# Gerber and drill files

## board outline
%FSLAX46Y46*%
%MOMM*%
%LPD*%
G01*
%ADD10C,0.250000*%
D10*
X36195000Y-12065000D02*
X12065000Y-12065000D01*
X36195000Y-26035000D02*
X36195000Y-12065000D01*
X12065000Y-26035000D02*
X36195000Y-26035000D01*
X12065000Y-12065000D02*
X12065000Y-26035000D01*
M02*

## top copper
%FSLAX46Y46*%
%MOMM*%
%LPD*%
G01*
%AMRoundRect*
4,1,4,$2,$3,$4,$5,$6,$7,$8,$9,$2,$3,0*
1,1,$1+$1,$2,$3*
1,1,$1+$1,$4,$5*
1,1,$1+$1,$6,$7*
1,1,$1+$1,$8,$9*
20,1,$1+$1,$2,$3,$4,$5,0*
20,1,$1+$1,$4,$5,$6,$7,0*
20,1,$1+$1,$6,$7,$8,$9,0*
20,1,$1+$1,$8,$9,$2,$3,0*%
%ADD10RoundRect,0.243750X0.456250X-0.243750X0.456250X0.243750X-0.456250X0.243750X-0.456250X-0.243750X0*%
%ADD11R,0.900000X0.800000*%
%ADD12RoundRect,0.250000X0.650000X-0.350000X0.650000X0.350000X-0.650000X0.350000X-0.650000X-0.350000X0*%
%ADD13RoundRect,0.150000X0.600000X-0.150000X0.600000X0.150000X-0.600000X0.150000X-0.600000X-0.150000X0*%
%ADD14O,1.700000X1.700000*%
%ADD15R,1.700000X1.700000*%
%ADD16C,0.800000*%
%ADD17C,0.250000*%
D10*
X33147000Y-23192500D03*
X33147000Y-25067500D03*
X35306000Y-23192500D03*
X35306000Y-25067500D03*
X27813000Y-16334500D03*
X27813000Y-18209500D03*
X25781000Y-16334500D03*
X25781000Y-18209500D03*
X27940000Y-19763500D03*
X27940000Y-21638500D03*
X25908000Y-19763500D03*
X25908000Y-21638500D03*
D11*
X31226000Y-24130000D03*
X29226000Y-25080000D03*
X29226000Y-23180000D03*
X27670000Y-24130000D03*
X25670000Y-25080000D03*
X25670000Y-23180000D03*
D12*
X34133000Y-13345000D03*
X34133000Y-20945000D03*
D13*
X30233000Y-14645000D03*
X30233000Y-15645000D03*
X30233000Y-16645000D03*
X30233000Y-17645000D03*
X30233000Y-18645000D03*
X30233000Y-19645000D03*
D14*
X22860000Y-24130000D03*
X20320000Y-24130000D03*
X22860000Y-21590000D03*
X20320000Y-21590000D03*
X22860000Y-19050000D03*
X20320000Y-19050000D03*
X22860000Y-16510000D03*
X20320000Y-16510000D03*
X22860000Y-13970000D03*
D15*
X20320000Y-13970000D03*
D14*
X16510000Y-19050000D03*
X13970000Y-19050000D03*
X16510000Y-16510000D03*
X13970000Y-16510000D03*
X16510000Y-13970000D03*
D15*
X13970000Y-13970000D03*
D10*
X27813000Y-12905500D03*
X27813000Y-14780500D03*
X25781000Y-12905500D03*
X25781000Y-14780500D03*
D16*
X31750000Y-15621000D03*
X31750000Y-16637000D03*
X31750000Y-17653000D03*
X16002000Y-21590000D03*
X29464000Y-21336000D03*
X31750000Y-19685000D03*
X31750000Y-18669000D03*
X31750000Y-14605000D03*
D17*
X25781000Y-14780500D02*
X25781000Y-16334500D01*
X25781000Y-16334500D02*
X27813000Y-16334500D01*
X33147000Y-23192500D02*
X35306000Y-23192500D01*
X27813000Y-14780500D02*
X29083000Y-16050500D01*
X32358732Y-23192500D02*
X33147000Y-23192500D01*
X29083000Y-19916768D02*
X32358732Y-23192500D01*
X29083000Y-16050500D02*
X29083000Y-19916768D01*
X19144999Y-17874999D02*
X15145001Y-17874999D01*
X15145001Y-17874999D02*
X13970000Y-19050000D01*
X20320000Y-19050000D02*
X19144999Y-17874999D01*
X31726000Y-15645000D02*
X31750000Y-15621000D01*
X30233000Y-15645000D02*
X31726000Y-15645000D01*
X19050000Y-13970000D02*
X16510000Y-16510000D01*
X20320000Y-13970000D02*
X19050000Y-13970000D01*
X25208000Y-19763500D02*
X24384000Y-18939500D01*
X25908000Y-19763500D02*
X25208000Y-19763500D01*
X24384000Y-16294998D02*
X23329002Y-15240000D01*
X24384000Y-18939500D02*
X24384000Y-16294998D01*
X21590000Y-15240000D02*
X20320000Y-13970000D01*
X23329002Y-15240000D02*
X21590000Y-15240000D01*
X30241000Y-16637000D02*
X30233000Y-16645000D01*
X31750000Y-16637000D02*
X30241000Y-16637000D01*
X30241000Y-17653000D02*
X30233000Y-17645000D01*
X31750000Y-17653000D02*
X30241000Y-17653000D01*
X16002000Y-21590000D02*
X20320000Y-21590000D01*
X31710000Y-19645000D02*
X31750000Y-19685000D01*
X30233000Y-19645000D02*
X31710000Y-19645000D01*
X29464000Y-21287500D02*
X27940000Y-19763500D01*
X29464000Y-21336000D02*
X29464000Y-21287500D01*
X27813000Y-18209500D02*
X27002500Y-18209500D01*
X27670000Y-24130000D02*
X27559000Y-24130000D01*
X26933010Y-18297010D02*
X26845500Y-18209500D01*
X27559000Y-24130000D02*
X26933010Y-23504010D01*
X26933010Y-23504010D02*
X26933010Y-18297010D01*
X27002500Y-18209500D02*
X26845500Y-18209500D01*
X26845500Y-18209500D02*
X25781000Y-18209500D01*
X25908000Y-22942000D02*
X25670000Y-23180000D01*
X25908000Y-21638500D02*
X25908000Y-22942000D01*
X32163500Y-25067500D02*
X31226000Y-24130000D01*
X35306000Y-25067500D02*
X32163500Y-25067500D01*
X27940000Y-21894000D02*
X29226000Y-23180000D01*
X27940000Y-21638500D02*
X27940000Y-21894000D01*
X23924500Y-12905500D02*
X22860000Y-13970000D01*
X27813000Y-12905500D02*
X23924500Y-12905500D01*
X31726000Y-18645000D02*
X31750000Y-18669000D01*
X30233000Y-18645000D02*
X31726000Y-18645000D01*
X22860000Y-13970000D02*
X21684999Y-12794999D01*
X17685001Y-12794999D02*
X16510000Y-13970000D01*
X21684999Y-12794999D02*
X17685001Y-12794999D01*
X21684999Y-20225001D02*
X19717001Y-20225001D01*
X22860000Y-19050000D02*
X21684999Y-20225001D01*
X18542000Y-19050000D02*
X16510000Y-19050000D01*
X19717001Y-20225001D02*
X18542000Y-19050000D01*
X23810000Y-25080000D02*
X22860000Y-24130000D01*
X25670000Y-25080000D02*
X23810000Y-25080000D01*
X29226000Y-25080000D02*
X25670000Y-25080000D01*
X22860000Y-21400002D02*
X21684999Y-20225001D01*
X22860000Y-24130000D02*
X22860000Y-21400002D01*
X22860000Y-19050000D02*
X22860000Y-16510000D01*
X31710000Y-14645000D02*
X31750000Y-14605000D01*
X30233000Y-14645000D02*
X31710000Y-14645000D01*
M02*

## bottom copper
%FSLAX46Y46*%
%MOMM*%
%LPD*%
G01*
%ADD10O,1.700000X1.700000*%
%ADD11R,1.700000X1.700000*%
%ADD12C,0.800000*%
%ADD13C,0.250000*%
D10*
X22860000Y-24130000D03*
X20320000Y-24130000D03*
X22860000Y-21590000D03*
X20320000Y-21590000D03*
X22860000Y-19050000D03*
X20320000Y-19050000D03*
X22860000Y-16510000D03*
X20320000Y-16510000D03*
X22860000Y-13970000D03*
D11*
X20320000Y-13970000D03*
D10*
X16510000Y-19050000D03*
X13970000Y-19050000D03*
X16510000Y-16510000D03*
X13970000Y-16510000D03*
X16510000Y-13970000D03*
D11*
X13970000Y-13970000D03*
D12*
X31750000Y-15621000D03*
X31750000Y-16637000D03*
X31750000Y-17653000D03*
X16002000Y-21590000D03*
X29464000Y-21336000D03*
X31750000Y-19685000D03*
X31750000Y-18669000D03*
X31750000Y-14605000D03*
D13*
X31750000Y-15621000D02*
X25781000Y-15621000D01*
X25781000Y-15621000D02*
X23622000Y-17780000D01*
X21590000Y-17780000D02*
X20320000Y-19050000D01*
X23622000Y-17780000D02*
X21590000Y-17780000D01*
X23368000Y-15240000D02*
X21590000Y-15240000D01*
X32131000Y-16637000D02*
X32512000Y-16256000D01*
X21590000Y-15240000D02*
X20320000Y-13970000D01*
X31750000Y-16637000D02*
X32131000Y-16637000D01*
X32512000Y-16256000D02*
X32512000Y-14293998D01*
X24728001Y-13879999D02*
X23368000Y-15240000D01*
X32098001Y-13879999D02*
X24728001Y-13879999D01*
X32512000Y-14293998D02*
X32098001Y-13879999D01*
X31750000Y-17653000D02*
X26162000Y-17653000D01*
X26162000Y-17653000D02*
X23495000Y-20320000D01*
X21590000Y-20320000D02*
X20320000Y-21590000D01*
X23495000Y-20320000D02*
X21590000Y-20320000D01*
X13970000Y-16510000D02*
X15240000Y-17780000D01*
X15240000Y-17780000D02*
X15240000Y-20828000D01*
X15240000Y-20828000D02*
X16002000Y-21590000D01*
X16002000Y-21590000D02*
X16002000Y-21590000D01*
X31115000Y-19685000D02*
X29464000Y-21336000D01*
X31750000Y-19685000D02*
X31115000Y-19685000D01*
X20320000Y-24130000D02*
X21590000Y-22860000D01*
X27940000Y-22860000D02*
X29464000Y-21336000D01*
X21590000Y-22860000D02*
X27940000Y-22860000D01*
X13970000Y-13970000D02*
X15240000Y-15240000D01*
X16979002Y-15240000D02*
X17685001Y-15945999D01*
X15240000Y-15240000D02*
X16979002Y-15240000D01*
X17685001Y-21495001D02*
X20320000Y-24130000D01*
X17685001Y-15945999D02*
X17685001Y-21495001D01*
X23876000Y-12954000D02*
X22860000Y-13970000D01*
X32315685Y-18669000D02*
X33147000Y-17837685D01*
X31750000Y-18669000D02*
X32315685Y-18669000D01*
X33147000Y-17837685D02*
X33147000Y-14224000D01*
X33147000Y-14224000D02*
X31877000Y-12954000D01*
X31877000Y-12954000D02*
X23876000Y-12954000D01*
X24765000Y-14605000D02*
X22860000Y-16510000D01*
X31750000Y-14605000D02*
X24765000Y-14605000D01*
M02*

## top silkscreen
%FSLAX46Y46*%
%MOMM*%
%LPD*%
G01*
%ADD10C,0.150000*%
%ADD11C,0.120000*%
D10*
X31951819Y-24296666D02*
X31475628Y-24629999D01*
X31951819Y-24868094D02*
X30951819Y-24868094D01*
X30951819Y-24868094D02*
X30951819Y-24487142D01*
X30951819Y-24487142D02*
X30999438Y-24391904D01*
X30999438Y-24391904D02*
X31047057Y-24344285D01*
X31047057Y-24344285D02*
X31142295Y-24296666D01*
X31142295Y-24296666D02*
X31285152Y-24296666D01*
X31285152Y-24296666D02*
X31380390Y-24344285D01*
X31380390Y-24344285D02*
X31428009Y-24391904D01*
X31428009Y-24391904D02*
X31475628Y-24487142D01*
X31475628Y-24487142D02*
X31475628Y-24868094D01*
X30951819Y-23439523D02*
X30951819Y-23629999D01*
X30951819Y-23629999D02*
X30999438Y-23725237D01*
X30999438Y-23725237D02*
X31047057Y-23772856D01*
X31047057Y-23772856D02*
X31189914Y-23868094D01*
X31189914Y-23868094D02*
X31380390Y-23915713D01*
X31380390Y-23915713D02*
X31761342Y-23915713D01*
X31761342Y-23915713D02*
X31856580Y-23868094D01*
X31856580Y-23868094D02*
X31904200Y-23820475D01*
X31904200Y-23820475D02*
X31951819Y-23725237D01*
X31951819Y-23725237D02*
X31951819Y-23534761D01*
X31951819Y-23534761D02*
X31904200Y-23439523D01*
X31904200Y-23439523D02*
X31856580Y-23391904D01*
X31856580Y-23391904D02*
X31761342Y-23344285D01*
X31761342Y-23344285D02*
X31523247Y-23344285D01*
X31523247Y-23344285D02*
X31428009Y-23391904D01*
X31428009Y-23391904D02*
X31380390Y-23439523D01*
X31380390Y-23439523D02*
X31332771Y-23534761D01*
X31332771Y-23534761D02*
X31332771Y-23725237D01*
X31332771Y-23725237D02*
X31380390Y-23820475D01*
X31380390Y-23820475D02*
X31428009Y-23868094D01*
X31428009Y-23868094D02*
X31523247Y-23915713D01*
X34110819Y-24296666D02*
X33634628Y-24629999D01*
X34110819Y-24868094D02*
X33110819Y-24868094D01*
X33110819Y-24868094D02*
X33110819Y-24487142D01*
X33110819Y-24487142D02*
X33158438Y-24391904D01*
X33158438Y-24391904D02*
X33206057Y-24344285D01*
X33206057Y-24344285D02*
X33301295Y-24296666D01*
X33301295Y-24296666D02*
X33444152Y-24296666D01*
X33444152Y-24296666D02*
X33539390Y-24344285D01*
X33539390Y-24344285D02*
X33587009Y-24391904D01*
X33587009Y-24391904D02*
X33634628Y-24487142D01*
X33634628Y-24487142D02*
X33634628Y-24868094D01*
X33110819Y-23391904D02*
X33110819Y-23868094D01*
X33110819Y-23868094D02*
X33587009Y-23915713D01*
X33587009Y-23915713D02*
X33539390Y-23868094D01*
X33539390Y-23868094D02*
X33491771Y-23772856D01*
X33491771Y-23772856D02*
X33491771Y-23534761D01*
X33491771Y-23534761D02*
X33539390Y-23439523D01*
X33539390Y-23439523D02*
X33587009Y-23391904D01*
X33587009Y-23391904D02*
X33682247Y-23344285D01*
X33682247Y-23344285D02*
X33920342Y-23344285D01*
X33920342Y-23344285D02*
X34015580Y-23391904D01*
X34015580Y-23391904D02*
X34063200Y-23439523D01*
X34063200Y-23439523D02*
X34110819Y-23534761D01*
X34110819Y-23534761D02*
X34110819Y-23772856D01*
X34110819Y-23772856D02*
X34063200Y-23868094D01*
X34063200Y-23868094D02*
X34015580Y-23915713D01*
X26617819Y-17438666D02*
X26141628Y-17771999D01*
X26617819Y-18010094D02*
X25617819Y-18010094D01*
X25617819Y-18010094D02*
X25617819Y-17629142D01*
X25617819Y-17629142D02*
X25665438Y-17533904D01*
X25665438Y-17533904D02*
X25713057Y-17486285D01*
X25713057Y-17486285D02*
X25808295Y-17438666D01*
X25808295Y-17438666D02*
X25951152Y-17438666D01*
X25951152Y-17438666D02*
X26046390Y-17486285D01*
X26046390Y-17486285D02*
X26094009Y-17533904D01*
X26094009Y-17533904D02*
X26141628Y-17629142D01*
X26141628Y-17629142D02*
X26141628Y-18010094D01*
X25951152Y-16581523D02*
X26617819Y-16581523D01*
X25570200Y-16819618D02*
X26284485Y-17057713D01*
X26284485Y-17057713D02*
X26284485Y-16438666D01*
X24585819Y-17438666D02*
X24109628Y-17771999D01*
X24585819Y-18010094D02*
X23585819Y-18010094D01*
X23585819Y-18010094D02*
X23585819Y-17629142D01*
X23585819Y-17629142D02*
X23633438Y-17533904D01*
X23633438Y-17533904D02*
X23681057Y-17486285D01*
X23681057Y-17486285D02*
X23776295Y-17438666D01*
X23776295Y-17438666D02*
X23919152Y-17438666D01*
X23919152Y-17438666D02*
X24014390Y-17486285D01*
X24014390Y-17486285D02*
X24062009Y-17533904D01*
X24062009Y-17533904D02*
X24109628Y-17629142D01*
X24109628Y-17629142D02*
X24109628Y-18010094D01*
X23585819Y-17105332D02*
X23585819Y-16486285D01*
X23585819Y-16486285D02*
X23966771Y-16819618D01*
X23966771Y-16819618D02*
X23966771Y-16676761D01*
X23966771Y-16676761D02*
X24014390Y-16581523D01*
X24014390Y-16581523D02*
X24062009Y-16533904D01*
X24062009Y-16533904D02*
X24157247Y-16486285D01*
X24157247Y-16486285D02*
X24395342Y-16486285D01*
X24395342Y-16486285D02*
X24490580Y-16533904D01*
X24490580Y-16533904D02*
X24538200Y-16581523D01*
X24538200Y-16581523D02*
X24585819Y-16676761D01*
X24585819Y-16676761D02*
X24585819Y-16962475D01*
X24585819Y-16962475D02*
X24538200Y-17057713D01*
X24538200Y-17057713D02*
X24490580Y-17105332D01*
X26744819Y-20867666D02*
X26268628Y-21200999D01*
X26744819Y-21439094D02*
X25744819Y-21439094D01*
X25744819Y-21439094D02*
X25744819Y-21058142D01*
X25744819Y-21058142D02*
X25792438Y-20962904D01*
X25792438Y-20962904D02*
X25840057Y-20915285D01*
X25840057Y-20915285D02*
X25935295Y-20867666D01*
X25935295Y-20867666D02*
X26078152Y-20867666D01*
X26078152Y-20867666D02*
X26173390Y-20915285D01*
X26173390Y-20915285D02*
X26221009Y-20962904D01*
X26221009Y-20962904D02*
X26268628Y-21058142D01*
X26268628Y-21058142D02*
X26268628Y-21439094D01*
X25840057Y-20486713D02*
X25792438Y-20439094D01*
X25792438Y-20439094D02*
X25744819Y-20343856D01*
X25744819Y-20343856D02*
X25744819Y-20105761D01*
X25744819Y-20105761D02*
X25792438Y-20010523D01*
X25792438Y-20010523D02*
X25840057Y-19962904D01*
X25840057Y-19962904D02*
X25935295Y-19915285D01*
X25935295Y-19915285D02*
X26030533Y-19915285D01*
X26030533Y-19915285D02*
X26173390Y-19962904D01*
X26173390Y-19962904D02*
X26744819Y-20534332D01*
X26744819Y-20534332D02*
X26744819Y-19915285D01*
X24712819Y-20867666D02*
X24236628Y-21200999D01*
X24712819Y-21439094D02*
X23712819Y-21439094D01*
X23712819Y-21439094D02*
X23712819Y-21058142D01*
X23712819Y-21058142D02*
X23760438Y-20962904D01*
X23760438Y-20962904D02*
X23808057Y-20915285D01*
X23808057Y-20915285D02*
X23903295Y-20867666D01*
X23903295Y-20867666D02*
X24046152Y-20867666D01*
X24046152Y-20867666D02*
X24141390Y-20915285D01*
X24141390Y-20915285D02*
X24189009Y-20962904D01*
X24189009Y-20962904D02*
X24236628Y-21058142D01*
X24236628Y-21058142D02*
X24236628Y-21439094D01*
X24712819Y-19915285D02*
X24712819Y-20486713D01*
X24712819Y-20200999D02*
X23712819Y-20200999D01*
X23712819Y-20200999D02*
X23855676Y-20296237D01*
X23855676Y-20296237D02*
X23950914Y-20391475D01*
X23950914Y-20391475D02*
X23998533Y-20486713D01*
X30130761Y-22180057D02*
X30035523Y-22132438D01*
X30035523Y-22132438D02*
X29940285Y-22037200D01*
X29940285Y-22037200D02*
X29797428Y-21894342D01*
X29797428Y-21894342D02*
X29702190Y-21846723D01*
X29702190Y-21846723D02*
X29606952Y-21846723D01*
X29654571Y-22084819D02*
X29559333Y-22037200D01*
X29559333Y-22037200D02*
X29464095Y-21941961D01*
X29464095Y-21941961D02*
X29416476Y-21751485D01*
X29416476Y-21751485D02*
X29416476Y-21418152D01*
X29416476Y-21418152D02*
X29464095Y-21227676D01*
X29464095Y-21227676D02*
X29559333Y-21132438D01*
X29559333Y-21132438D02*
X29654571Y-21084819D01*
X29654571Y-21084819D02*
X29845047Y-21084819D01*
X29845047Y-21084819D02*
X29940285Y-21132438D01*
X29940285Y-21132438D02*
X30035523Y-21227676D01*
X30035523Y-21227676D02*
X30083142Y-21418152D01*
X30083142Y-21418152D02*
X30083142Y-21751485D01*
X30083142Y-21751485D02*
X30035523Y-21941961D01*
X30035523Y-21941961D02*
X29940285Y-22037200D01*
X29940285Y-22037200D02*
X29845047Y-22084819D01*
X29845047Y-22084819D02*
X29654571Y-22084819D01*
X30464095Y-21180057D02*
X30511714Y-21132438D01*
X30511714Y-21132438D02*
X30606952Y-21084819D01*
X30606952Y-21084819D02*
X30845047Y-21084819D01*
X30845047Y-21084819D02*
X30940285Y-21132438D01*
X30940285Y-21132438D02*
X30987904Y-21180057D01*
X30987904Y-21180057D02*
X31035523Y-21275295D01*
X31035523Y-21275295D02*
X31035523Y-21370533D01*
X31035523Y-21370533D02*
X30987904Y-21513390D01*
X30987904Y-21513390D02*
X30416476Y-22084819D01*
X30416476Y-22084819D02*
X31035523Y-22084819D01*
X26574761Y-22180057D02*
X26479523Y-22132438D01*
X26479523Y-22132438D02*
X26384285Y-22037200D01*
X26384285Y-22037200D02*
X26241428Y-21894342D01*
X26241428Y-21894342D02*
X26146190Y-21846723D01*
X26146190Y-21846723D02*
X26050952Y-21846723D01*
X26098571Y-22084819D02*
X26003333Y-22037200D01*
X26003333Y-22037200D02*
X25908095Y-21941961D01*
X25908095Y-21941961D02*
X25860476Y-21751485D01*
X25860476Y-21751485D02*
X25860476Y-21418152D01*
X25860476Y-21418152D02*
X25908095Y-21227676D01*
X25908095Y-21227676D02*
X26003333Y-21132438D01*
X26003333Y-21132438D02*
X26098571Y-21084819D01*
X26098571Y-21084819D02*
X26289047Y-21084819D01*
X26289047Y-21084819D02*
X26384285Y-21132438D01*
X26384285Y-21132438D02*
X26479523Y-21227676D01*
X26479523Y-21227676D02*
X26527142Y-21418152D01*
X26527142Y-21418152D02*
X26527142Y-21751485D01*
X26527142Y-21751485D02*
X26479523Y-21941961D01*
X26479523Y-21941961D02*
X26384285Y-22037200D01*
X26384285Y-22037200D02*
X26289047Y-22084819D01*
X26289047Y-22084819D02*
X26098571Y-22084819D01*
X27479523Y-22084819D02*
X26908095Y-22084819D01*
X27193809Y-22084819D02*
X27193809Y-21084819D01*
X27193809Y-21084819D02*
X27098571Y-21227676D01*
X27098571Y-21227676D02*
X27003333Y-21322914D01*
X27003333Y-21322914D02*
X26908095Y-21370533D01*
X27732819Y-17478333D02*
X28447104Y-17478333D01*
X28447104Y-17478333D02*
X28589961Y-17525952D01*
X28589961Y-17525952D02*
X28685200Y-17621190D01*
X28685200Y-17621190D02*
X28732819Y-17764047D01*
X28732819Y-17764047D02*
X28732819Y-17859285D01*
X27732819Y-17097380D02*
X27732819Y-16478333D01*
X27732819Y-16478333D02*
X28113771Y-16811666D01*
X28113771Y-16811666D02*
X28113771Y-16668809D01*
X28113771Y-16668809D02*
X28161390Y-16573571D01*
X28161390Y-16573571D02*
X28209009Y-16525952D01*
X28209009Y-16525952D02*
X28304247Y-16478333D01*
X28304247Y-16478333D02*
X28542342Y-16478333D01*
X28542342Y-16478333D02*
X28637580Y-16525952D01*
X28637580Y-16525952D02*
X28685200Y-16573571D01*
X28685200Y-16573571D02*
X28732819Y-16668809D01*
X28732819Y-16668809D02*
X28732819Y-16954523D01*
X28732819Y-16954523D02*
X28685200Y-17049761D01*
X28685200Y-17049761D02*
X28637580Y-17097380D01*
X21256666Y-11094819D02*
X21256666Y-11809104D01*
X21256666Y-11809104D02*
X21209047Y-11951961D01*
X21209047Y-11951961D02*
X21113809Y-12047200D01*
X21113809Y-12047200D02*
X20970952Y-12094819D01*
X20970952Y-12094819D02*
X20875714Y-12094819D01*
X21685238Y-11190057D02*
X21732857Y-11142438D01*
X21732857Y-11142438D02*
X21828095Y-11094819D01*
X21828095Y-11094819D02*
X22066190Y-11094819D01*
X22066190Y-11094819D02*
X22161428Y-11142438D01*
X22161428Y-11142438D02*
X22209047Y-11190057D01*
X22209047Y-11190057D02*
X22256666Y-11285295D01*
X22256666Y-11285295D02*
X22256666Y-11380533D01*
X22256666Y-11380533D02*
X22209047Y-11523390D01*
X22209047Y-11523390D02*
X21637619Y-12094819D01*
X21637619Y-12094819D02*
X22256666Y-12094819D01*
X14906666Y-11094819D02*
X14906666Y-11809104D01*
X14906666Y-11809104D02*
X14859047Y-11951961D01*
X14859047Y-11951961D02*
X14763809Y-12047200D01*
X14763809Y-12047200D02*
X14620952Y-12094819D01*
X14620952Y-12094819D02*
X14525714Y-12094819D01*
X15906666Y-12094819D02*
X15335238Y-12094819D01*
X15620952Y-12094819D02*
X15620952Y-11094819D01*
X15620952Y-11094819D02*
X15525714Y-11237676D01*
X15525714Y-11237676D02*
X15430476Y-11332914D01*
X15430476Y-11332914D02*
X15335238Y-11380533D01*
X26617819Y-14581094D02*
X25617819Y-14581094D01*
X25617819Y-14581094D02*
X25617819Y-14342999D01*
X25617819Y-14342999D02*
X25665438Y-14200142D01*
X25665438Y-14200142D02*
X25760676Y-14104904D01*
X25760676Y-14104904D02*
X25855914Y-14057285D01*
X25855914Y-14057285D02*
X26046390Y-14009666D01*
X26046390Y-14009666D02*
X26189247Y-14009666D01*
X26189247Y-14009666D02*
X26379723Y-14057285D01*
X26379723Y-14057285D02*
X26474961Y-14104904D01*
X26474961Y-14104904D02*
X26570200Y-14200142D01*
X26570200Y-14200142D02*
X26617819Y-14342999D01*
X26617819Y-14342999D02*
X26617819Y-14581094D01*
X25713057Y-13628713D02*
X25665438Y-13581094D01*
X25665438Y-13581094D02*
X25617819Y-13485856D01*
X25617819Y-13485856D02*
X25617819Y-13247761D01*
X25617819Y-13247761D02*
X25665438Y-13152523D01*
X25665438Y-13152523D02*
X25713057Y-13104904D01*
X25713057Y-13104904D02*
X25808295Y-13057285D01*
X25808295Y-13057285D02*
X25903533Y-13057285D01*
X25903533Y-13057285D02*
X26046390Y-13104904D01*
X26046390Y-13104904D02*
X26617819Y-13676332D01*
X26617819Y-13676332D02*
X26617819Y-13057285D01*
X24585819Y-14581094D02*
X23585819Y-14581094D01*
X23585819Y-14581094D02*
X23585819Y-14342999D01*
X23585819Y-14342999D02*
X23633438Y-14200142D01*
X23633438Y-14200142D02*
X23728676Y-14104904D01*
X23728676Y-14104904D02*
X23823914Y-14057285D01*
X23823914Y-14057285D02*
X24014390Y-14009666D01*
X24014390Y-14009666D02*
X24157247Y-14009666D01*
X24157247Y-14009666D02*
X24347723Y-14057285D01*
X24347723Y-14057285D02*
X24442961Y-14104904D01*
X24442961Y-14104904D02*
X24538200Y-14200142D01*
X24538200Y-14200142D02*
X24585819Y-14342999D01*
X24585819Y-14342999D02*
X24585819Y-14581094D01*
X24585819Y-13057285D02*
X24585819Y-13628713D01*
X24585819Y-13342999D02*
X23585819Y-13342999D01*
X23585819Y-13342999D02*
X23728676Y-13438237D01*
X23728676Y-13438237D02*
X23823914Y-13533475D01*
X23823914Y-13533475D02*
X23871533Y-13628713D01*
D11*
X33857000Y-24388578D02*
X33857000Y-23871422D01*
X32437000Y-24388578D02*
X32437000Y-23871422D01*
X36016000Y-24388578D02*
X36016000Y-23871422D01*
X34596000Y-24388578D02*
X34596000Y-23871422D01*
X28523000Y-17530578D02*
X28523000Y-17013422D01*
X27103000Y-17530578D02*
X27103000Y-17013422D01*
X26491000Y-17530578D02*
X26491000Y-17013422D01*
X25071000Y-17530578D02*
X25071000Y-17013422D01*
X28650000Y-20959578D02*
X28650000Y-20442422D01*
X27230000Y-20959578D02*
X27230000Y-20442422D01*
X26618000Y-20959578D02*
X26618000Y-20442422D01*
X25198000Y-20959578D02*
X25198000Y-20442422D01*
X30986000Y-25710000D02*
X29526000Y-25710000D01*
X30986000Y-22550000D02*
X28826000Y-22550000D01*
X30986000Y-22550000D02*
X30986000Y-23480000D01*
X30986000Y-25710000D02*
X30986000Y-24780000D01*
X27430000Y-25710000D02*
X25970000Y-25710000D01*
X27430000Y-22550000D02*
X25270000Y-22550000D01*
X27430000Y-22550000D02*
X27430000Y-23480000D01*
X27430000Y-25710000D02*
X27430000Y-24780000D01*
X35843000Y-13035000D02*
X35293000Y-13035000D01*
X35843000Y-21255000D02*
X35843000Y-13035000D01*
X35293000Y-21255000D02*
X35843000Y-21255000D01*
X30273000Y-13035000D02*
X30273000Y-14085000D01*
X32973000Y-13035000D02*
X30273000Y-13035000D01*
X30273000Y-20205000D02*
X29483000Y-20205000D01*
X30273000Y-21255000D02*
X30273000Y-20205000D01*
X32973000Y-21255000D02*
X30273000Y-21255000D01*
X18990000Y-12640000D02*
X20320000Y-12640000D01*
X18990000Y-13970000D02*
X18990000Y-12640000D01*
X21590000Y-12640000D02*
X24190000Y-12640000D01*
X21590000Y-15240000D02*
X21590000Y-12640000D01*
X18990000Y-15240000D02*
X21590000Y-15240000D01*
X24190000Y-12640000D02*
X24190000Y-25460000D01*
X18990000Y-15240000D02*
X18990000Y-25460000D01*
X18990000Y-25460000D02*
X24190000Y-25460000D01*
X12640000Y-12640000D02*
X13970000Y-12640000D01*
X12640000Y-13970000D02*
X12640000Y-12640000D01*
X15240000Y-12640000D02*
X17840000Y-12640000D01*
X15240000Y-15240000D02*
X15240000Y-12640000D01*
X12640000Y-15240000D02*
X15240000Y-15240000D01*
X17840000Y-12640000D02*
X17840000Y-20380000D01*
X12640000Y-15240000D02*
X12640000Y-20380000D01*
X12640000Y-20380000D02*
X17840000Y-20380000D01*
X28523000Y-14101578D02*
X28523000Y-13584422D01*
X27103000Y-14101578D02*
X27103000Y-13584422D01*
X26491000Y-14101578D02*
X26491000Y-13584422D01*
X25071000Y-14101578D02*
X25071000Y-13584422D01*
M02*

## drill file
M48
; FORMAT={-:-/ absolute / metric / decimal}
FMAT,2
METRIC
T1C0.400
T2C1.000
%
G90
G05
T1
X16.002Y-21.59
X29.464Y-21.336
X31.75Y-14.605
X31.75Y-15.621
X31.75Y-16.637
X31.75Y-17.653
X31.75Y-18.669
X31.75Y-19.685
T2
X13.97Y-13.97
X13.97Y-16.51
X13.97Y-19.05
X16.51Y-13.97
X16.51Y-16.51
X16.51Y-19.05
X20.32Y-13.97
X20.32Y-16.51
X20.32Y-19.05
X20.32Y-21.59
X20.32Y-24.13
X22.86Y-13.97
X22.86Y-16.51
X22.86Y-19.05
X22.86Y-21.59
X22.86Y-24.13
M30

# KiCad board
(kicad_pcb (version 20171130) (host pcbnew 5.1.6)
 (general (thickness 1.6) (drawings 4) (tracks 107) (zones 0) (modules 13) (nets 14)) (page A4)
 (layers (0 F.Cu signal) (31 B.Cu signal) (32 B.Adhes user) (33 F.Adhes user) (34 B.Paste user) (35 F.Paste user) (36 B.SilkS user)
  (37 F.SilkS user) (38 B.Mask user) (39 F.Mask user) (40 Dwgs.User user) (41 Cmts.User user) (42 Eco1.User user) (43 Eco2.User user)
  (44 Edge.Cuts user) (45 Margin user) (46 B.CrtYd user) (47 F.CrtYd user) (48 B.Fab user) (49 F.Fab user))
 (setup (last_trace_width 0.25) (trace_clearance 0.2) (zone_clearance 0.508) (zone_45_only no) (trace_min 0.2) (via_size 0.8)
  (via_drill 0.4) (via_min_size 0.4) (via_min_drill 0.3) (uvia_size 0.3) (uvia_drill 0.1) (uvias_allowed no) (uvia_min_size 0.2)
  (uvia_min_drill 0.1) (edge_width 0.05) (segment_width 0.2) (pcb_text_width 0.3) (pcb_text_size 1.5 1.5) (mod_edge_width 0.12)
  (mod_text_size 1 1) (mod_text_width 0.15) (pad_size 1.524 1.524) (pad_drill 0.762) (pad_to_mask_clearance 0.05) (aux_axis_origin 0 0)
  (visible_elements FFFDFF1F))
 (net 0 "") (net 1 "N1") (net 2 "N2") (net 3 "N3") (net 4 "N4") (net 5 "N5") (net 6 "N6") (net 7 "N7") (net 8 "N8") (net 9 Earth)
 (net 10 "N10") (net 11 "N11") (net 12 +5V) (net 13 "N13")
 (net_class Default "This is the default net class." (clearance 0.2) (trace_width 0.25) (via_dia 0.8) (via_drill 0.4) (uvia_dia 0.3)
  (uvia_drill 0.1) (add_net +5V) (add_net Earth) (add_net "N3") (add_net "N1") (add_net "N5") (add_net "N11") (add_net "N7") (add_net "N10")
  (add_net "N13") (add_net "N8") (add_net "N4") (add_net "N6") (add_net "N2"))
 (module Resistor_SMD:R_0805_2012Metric (layer F.Cu) (at 33.147 24.13 90)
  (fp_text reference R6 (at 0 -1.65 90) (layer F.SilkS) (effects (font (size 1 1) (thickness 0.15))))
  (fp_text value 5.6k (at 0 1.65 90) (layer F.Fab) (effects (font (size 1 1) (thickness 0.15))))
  (fp_line (start -0.258578 0.71) (end 0.258578 0.71) (layer F.SilkS) (width 0.12))
  (fp_line (start -0.258578 -0.71) (end 0.258578 -0.71) (layer F.SilkS) (width 0.12))
  (pad 2 smd roundrect (at 0.9375 0 90) (size 0.975 1.4) (layers F.Cu F.Paste F.Mask) (roundrect_rratio 0.25) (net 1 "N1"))
  (pad 1 smd roundrect (at -0.9375 0 90) (size 0.975 1.4) (layers F.Cu F.Paste F.Mask) (roundrect_rratio 0.25) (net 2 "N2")))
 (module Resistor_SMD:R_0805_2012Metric (layer F.Cu) (at 35.306 24.13 90)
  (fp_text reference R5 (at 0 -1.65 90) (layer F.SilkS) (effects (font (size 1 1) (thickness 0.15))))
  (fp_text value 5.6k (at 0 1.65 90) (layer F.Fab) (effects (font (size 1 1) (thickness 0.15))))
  (fp_line (start -0.258578 0.71) (end 0.258578 0.71) (layer F.SilkS) (width 0.12))
  (fp_line (start -0.258578 -0.71) (end 0.258578 -0.71) (layer F.SilkS) (width 0.12))
  (pad 2 smd roundrect (at 0.9375 0 90) (size 0.975 1.4) (layers F.Cu F.Paste F.Mask) (roundrect_rratio 0.25) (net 1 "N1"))
  (pad 1 smd roundrect (at -0.9375 0 90) (size 0.975 1.4) (layers F.Cu F.Paste F.Mask) (roundrect_rratio 0.25) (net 2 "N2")))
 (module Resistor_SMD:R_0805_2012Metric (layer F.Cu) (at 27.813 17.272 90)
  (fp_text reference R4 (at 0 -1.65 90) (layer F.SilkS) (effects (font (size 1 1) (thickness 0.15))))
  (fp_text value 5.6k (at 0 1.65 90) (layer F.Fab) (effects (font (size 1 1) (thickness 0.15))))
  (fp_line (start -0.258578 0.71) (end 0.258578 0.71) (layer F.SilkS) (width 0.12))
  (fp_line (start -0.258578 -0.71) (end 0.258578 -0.71) (layer F.SilkS) (width 0.12))
  (pad 2 smd roundrect (at 0.9375 0 90) (size 0.975 1.4) (layers F.Cu F.Paste F.Mask) (roundrect_rratio 0.25) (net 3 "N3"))
  (pad 1 smd roundrect (at -0.9375 0 90) (size 0.975 1.4) (layers F.Cu F.Paste F.Mask) (roundrect_rratio 0.25) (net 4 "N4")))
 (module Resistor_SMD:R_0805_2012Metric (layer F.Cu) (at 25.781 17.272 90)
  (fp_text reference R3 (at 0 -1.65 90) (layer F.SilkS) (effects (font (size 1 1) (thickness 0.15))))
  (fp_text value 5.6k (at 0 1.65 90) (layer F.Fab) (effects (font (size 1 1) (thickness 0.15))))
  (fp_line (start -0.258578 0.71) (end 0.258578 0.71) (layer F.SilkS) (width 0.12))
  (fp_line (start -0.258578 -0.71) (end 0.258578 -0.71) (layer F.SilkS) (width 0.12))
  (pad 2 smd roundrect (at 0.9375 0 90) (size 0.975 1.4) (layers F.Cu F.Paste F.Mask) (roundrect_rratio 0.25) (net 3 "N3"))
  (pad 1 smd roundrect (at -0.9375 0 90) (size 0.975 1.4) (layers F.Cu F.Paste F.Mask) (roundrect_rratio 0.25) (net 4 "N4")))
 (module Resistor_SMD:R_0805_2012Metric (layer F.Cu) (at 27.94 20.701 90)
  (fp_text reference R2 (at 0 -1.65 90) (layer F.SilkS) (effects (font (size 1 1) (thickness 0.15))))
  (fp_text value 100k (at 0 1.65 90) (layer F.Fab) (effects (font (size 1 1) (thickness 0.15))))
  (fp_line (start -0.258578 0.71) (end 0.258578 0.71) (layer F.SilkS) (width 0.12))
  (fp_line (start -0.258578 -0.71) (end 0.258578 -0.71) (layer F.SilkS) (width 0.12))
  (pad 2 smd roundrect (at 0.9375 0 90) (size 0.975 1.4) (layers F.Cu F.Paste F.Mask) (roundrect_rratio 0.25) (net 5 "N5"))
  (pad 1 smd roundrect (at -0.9375 0 90) (size 0.975 1.4) (layers F.Cu F.Paste F.Mask) (roundrect_rratio 0.25) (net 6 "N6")))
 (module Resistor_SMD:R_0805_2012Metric (layer F.Cu) (at 25.908 20.701 90)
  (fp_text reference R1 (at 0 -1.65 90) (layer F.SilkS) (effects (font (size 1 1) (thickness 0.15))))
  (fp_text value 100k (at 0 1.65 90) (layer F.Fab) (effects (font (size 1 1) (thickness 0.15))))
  (fp_line (start -0.258578 0.71) (end 0.258578 0.71) (layer F.SilkS) (width 0.12))
  (fp_line (start -0.258578 -0.71) (end 0.258578 -0.71) (layer F.SilkS) (width 0.12))
  (pad 2 smd roundrect (at 0.9375 0 90) (size 0.975 1.4) (layers F.Cu F.Paste F.Mask) (roundrect_rratio 0.25) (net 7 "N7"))
  (pad 1 smd roundrect (at -0.9375 0 90) (size 0.975 1.4) (layers F.Cu F.Paste F.Mask) (roundrect_rratio 0.25) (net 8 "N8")))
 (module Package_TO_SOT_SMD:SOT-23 (layer F.Cu) (at 30.226 24.13)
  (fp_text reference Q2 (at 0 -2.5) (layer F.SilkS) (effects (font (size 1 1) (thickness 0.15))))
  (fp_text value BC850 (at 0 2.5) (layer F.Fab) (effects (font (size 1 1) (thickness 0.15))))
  (fp_line (start 0.76 1.58) (end -0.7 1.58) (layer F.SilkS) (width 0.12))
  (fp_line (start 0.76 -1.58) (end -1.4 -1.58) (layer F.SilkS) (width 0.12))
  (fp_line (start 0.76 -1.58) (end 0.76 -0.65) (layer F.SilkS) (width 0.12))
  (fp_line (start 0.76 1.58) (end 0.76 0.65) (layer F.SilkS) (width 0.12))
  (pad 3 smd rect (at 1 0) (size 0.9 0.8) (layers F.Cu F.Paste F.Mask) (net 2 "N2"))
  (pad 2 smd rect (at -1 0.95) (size 0.9 0.8) (layers F.Cu F.Paste F.Mask) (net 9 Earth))
  (pad 1 smd rect (at -1 -0.95) (size 0.9 0.8) (layers F.Cu F.Paste F.Mask) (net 6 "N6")))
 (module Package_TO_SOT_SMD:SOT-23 (layer F.Cu) (at 26.67 24.13)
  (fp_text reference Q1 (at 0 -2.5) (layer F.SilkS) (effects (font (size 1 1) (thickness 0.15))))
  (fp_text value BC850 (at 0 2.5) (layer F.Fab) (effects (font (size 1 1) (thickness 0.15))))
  (fp_line (start 0.76 1.58) (end -0.7 1.58) (layer F.SilkS) (width 0.12))
  (fp_line (start 0.76 -1.58) (end -1.4 -1.58) (layer F.SilkS) (width 0.12))
  (fp_line (start 0.76 -1.58) (end 0.76 -0.65) (layer F.SilkS) (width 0.12))
  (fp_line (start 0.76 1.58) (end 0.76 0.65) (layer F.SilkS) (width 0.12))
  (pad 3 smd rect (at 1 0) (size 0.9 0.8) (layers F.Cu F.Paste F.Mask) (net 4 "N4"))
  (pad 2 smd rect (at -1 0.95) (size 0.9 0.8) (layers F.Cu F.Paste F.Mask) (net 9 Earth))
  (pad 1 smd rect (at -1 -0.95) (size 0.9 0.8) (layers F.Cu F.Paste F.Mask) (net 8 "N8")))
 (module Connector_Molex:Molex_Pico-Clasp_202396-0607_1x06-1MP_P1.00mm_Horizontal (layer F.Cu) (at 32.258 17.145 90)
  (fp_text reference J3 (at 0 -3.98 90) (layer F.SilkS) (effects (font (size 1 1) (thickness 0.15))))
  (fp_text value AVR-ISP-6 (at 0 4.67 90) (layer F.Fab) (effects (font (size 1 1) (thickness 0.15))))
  (fp_line (start 4.11 3.585) (end 4.11 3.035) (layer F.SilkS) (width 0.12))
  (fp_line (start -4.11 3.585) (end 4.11 3.585) (layer F.SilkS) (width 0.12))
  (fp_line (start -4.11 3.035) (end -4.11 3.585) (layer F.SilkS) (width 0.12))
  (fp_line (start 4.11 -1.985) (end 3.06 -1.985) (layer F.SilkS) (width 0.12))
  (fp_line (start 4.11 0.715) (end 4.11 -1.985) (layer F.SilkS) (width 0.12))
  (fp_line (start -3.06 -1.985) (end -3.06 -2.775) (layer F.SilkS) (width 0.12))
  (fp_line (start -4.11 -1.985) (end -3.06 -1.985) (layer F.SilkS) (width 0.12))
  (fp_line (start -4.11 0.715) (end -4.11 -1.985) (layer F.SilkS) (width 0.12))
  (pad MP smd roundrect (at 3.8 1.875 90) (size 1.2 1.8) (layers F.Cu F.Paste F.Mask) (roundrect_rratio 0.208333))
  (pad MP smd roundrect (at -3.8 1.875 90) (size 1.2 1.8) (layers F.Cu F.Paste F.Mask) (roundrect_rratio 0.208333))
  (pad 6 smd roundrect (at 2.5 -2.025 90) (size 0.6 1.5) (layers F.Cu F.Paste F.Mask) (roundrect_rratio 0.25) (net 9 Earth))
  (pad 5 smd roundrect (at 1.5 -2.025 90) (size 0.6 1.5) (layers F.Cu F.Paste F.Mask) (roundrect_rratio 0.25) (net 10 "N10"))
  (pad 4 smd roundrect (at 0.5 -2.025 90) (size 0.6 1.5) (layers F.Cu F.Paste F.Mask) (roundrect_rratio 0.25) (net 7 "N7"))
  (pad 3 smd roundrect (at -0.5 -2.025 90) (size 0.6 1.5) (layers F.Cu F.Paste F.Mask) (roundrect_rratio 0.25) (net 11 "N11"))
  (pad 2 smd roundrect (at -1.5 -2.025 90) (size 0.6 1.5) (layers F.Cu F.Paste F.Mask) (roundrect_rratio 0.25) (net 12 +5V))
  (pad 1 smd roundrect (at -2.5 -2.025 90) (size 0.6 1.5) (layers F.Cu F.Paste F.Mask) (roundrect_rratio 0.25) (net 5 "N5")))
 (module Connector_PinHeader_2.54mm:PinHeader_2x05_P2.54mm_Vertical (layer F.Cu) (at 20.32 13.97)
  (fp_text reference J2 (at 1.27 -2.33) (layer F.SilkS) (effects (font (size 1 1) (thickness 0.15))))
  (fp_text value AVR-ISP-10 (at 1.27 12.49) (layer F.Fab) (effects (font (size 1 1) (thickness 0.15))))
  (fp_line (start -1.33 -1.33) (end 0 -1.33) (layer F.SilkS) (width 0.12))
  (fp_line (start -1.33 0) (end -1.33 -1.33) (layer F.SilkS) (width 0.12))
  (fp_line (start 1.27 -1.33) (end 3.87 -1.33) (layer F.SilkS) (width 0.12))
  (fp_line (start 1.27 1.27) (end 1.27 -1.33) (layer F.SilkS) (width 0.12))
  (fp_line (start -1.33 1.27) (end 1.27 1.27) (layer F.SilkS) (width 0.12))
  (fp_line (start 3.87 -1.33) (end 3.87 11.49) (layer F.SilkS) (width 0.12))
  (fp_line (start -1.33 1.27) (end -1.33 11.49) (layer F.SilkS) (width 0.12))
  (fp_line (start -1.33 11.49) (end 3.87 11.49) (layer F.SilkS) (width 0.12))
  (pad 10 thru_hole oval (at 2.54 10.16) (size 1.7 1.7) (drill 1) (layers *.Cu *.Mask) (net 9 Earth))
  (pad 9 thru_hole oval (at 0 10.16) (size 1.7 1.7) (drill 1) (layers *.Cu *.Mask) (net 5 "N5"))
  (pad 8 thru_hole oval (at 2.54 7.62) (size 1.7 1.7) (drill 1) (layers *.Cu *.Mask) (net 9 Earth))
  (pad 7 thru_hole oval (at 0 7.62) (size 1.7 1.7) (drill 1) (layers *.Cu *.Mask) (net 11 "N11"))
  (pad 6 thru_hole oval (at 2.54 5.08) (size 1.7 1.7) (drill 1) (layers *.Cu *.Mask) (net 9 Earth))
  (pad 5 thru_hole oval (at 0 5.08) (size 1.7 1.7) (drill 1) (layers *.Cu *.Mask) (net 10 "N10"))
  (pad 4 thru_hole oval (at 2.54 2.54) (size 1.7 1.7) (drill 1) (layers *.Cu *.Mask) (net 9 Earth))
  (pad 3 thru_hole oval (at 0 2.54) (size 1.7 1.7) (drill 1) (layers *.Cu *.Mask) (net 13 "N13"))
  (pad 2 thru_hole oval (at 2.54 0) (size 1.7 1.7) (drill 1) (layers *.Cu *.Mask) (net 12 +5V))
  (pad 1 thru_hole rect (at 0 0) (size 1.7 1.7) (drill 1) (layers *.Cu *.Mask) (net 7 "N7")))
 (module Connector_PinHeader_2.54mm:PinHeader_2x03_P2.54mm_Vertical (layer F.Cu) (at 13.97 13.97)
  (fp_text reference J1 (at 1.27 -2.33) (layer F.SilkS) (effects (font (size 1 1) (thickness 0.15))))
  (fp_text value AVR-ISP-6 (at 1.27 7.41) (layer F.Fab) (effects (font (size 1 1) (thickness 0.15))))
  (fp_line (start -1.33 -1.33) (end 0 -1.33) (layer F.SilkS) (width 0.12))
  (fp_line (start -1.33 0) (end -1.33 -1.33) (layer F.SilkS) (width 0.12))
  (fp_line (start 1.27 -1.33) (end 3.87 -1.33) (layer F.SilkS) (width 0.12))
  (fp_line (start 1.27 1.27) (end 1.27 -1.33) (layer F.SilkS) (width 0.12))
  (fp_line (start -1.33 1.27) (end 1.27 1.27) (layer F.SilkS) (width 0.12))
  (fp_line (start 3.87 -1.33) (end 3.87 6.41) (layer F.SilkS) (width 0.12))
  (fp_line (start -1.33 1.27) (end -1.33 6.41) (layer F.SilkS) (width 0.12))
  (fp_line (start -1.33 6.41) (end 3.87 6.41) (layer F.SilkS) (width 0.12))
  (pad 6 thru_hole oval (at 2.54 5.08) (size 1.7 1.7) (drill 1) (layers *.Cu *.Mask) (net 9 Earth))
  (pad 5 thru_hole oval (at 0 5.08) (size 1.7 1.7) (drill 1) (layers *.Cu *.Mask) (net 10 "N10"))
  (pad 4 thru_hole oval (at 2.54 2.54) (size 1.7 1.7) (drill 1) (layers *.Cu *.Mask) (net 7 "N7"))
  (pad 3 thru_hole oval (at 0 2.54) (size 1.7 1.7) (drill 1) (layers *.Cu *.Mask) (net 11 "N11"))
  (pad 2 thru_hole oval (at 2.54 0) (size 1.7 1.7) (drill 1) (layers *.Cu *.Mask) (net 12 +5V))
  (pad 1 thru_hole rect (at 0 0) (size 1.7 1.7) (drill 1) (layers *.Cu *.Mask) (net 5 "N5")))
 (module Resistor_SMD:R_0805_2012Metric (layer F.Cu) (at 27.813 13.843 90)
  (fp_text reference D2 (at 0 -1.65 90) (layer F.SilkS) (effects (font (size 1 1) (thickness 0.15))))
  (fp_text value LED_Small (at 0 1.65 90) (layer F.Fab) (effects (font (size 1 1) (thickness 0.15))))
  (fp_line (start -0.258578 0.71) (end 0.258578 0.71) (layer F.SilkS) (width 0.12))
  (fp_line (start -0.258578 -0.71) (end 0.258578 -0.71) (layer F.SilkS) (width 0.12))
  (pad 2 smd roundrect (at 0.9375 0 90) (size 0.975 1.4) (layers F.Cu F.Paste F.Mask) (roundrect_rratio 0.25) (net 12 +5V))
  (pad 1 smd roundrect (at -0.9375 0 90) (size 0.975 1.4) (layers F.Cu F.Paste F.Mask) (roundrect_rratio 0.25) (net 1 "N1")))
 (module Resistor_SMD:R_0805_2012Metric (layer F.Cu) (at 25.781 13.843 90)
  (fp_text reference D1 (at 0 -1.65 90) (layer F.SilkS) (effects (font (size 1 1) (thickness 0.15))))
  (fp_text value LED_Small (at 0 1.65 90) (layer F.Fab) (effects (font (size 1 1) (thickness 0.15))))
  (fp_line (start -0.258578 0.71) (end 0.258578 0.71) (layer F.SilkS) (width 0.12))
  (fp_line (start -0.258578 -0.71) (end 0.258578 -0.71) (layer F.SilkS) (width 0.12))
  (pad 2 smd roundrect (at 0.9375 0 90) (size 0.975 1.4) (layers F.Cu F.Paste F.Mask) (roundrect_rratio 0.25) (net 12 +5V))
  (pad 1 smd roundrect (at -0.9375 0 90) (size 0.975 1.4) (layers F.Cu F.Paste F.Mask) (roundrect_rratio 0.25) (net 3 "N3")))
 (gr_line (start 36.195 12.065) (end 12.065 12.065) (layer Edge.Cuts) (width 0.25))
 (gr_line (start 36.195 26.035) (end 36.195 12.065) (layer Edge.Cuts) (width 0.25))
 (gr_line (start 12.065 26.035) (end 36.195 26.035) (layer Edge.Cuts) (width 0.25))
 (gr_line (start 12.065 12.065) (end 12.065 26.035) (layer Edge.Cuts) (width 0.25))
 (segment (start 25.781 14.7805) (end 25.781 16.3345) (width 0.25) (layer F.Cu) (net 3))
 (segment (start 25.781 16.3345) (end 27.813 16.3345) (width 0.25) (layer F.Cu) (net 3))
 (segment (start 33.147 23.1925) (end 35.306 23.1925) (width 0.25) (layer F.Cu) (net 1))
 (segment (start 27.813 14.7805) (end 29.083 16.0505) (width 0.25) (layer F.Cu) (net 1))
 (segment (start 32.358732 23.1925) (end 33.147 23.1925) (width 0.25) (layer F.Cu) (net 1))
 (segment (start 29.083 19.916768) (end 32.358732 23.1925) (width 0.25) (layer F.Cu) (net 1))
 (segment (start 29.083 16.0505) (end 29.083 19.916768) (width 0.25) (layer F.Cu) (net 1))
 (via (at 31.75 15.621) (size 0.8) (drill 0.4) (layers F.Cu B.Cu) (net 10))
 (segment (start 19.144999 17.874999) (end 15.145001 17.874999) (width 0.25) (layer F.Cu) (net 10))
 (segment (start 15.145001 17.874999) (end 13.97 19.05) (width 0.25) (layer F.Cu) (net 10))
 (segment (start 20.32 19.05) (end 19.144999 17.874999) (width 0.25) (layer F.Cu) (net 10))
 (segment (start 31.726 15.645) (end 31.75 15.621) (width 0.25) (layer F.Cu) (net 10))
 (segment (start 30.233 15.645) (end 31.726 15.645) (width 0.25) (layer F.Cu) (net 10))
 (segment (start 31.75 15.621) (end 25.781 15.621) (width 0.25) (layer B.Cu) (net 10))
 (segment (start 25.781 15.621) (end 23.622 17.78) (width 0.25) (layer B.Cu) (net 10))
 (segment (start 21.59 17.78) (end 20.32 19.05) (width 0.25) (layer B.Cu) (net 10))
 (segment (start 23.622 17.78) (end 21.59 17.78) (width 0.25) (layer B.Cu) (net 10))
 (via (at 31.75 16.637) (size 0.8) (drill 0.4) (layers F.Cu B.Cu) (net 7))
 (segment (start 19.05 13.97) (end 16.51 16.51) (width 0.25) (layer F.Cu) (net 7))
 (segment (start 20.32 13.97) (end 19.05 13.97) (width 0.25) (layer F.Cu) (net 7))
 (segment (start 25.208 19.7635) (end 24.384 18.9395) (width 0.25) (layer F.Cu) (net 7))
 (segment (start 25.908 19.7635) (end 25.208 19.7635) (width 0.25) (layer F.Cu) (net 7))
 (segment (start 24.384 16.294998) (end 23.329002 15.24) (width 0.25) (layer F.Cu) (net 7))
 (segment (start 24.384 18.9395) (end 24.384 16.294998) (width 0.25) (layer F.Cu) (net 7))
 (segment (start 21.59 15.24) (end 20.32 13.97) (width 0.25) (layer F.Cu) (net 7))
 (segment (start 23.329002 15.24) (end 21.59 15.24) (width 0.25) (layer F.Cu) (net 7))
 (segment (start 30.241 16.637) (end 30.233 16.645) (width 0.25) (layer F.Cu) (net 7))
 (segment (start 31.75 16.637) (end 30.241 16.637) (width 0.25) (layer F.Cu) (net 7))
 (segment (start 23.368 15.24) (end 21.59 15.24) (width 0.25) (layer B.Cu) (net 7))
 (segment (start 32.131 16.637) (end 32.512 16.256) (width 0.25) (layer B.Cu) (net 7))
 (segment (start 21.59 15.24) (end 20.32 13.97) (width 0.25) (layer B.Cu) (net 7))
 (segment (start 31.75 16.637) (end 32.131 16.637) (width 0.25) (layer B.Cu) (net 7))
 (segment (start 32.512 16.256) (end 32.512 14.293998) (width 0.25) (layer B.Cu) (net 7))
 (segment (start 24.728001 13.879999) (end 23.368 15.24) (width 0.25) (layer B.Cu) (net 7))
 (segment (start 32.098001 13.879999) (end 24.728001 13.879999) (width 0.25) (layer B.Cu) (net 7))
 (segment (start 32.512 14.293998) (end 32.098001 13.879999) (width 0.25) (layer B.Cu) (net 7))
 (via (at 31.75 17.653) (size 0.8) (drill 0.4) (layers F.Cu B.Cu) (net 11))
 (segment (start 31.75 17.653) (end 26.162 17.653) (width 0.25) (layer B.Cu) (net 11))
 (segment (start 26.162 17.653) (end 23.495 20.32) (width 0.25) (layer B.Cu) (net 11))
 (segment (start 21.59 20.32) (end 20.32 21.59) (width 0.25) (layer B.Cu) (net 11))
 (segment (start 23.495 20.32) (end 21.59 20.32) (width 0.25) (layer B.Cu) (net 11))
 (segment (start 30.241 17.653) (end 30.233 17.645) (width 0.25) (layer F.Cu) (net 11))
 (segment (start 31.75 17.653) (end 30.241 17.653) (width 0.25) (layer F.Cu) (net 11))
 (segment (start 13.97 16.51) (end 15.24 17.78) (width 0.25) (layer B.Cu) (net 11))
 (segment (start 15.24 17.78) (end 15.24 20.828) (width 0.25) (layer B.Cu) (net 11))
 (segment (start 15.24 20.828) (end 16.002 21.59) (width 0.25) (layer B.Cu) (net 11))
 (segment (start 16.002 21.59) (end 16.002 21.59) (width 0.25) (layer B.Cu) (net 11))
 (via (at 16.002 21.59) (size 0.8) (drill 0.4) (layers F.Cu B.Cu) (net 11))
 (segment (start 16.002 21.59) (end 20.32 21.59) (width 0.25) (layer F.Cu) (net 11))
 (via (at 29.464 21.336) (size 0.8) (drill 0.4) (layers F.Cu B.Cu) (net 5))
 (via (at 31.75 19.685) (size 0.8) (drill 0.4) (layers F.Cu B.Cu) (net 5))
 (segment (start 31.71 19.645) (end 31.75 19.685) (width 0.25) (layer F.Cu) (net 5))
 (segment (start 30.233 19.645) (end 31.71 19.645) (width 0.25) (layer F.Cu) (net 5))
 (segment (start 29.464 21.2875) (end 27.94 19.7635) (width 0.25) (layer F.Cu) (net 5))
 (segment (start 29.464 21.336) (end 29.464 21.2875) (width 0.25) (layer F.Cu) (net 5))
 (segment (start 31.115 19.685) (end 29.464 21.336) (width 0.25) (layer B.Cu) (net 5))
 (segment (start 31.75 19.685) (end 31.115 19.685) (width 0.25) (layer B.Cu) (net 5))
 (segment (start 20.32 24.13) (end 21.59 22.86) (width 0.25) (layer B.Cu) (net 5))
 (segment (start 27.94 22.86) (end 29.464 21.336) (width 0.25) (layer B.Cu) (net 5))
 (segment (start 21.59 22.86) (end 27.94 22.86) (width 0.25) (layer B.Cu) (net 5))
 (segment (start 13.97 13.97) (end 15.24 15.24) (width 0.25) (layer B.Cu) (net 5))
 (segment (start 16.979002 15.24) (end 17.685001 15.945999) (width 0.25) (layer B.Cu) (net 5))
 (segment (start 15.24 15.24) (end 16.979002 15.24) (width 0.25) (layer B.Cu) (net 5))
 (segment (start 17.685001 21.495001) (end 20.32 24.13) (width 0.25) (layer B.Cu) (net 5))
 (segment (start 17.685001 15.945999) (end 17.685001 21.495001) (width 0.25) (layer B.Cu) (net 5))
 (segment (start 27.813 18.2095) (end 27.0025 18.2095) (width 0.25) (layer F.Cu) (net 4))
 (segment (start 27.67 24.13) (end 27.559 24.13) (width 0.25) (layer F.Cu) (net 4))
 (segment (start 26.93301 18.29701) (end 26.8455 18.2095) (width 0.25) (layer F.Cu) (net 4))
 (segment (start 27.559 24.13) (end 26.93301 23.50401) (width 0.25) (layer F.Cu) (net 4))
 (segment (start 26.93301 23.50401) (end 26.93301 18.29701) (width 0.25) (layer F.Cu) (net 4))
 (segment (start 27.0025 18.2095) (end 26.8455 18.2095) (width 0.25) (layer F.Cu) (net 4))
 (segment (start 26.8455 18.2095) (end 25.781 18.2095) (width 0.25) (layer F.Cu) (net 4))
 (segment (start 25.908 22.942) (end 25.67 23.18) (width 0.25) (layer F.Cu) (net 8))
 (segment (start 25.908 21.6385) (end 25.908 22.942) (width 0.25) (layer F.Cu) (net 8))
 (segment (start 32.1635 25.0675) (end 31.226 24.13) (width 0.25) (layer F.Cu) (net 2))
 (segment (start 35.306 25.0675) (end 32.1635 25.0675) (width 0.25) (layer F.Cu) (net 2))
 (segment (start 27.94 21.894) (end 29.226 23.18) (width 0.25) (layer F.Cu) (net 6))
 (segment (start 27.94 21.6385) (end 27.94 21.894) (width 0.25) (layer F.Cu) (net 6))
 (via (at 31.75 18.669) (size 0.8) (drill 0.4) (layers F.Cu B.Cu) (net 12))
 (segment (start 23.9245 12.9055) (end 22.86 13.97) (width 0.25) (layer F.Cu) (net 12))
 (segment (start 27.813 12.9055) (end 23.9245 12.9055) (width 0.25) (layer F.Cu) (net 12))
 (segment (start 23.876 12.954) (end 22.86 13.97) (width 0.25) (layer B.Cu) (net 12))
 (segment (start 32.315685 18.669) (end 33.147 17.837685) (width 0.25) (layer B.Cu) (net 12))
 (segment (start 31.75 18.669) (end 32.315685 18.669) (width 0.25) (layer B.Cu) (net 12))
 (segment (start 33.147 17.837685) (end 33.147 14.224) (width 0.25) (layer B.Cu) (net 12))
 (segment (start 33.147 14.224) (end 31.877 12.954) (width 0.25) (layer B.Cu) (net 12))
 (segment (start 31.877 12.954) (end 23.876 12.954) (width 0.25) (layer B.Cu) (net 12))
 (segment (start 31.726 18.645) (end 31.75 18.669) (width 0.25) (layer F.Cu) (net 12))
 (segment (start 30.233 18.645) (end 31.726 18.645) (width 0.25) (layer F.Cu) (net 12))
 (segment (start 22.86 13.97) (end 21.684999 12.794999) (width 0.25) (layer F.Cu) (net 12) (status 1000000))
 (segment (start 17.685001 12.794999) (end 16.51 13.97) (width 0.25) (layer F.Cu) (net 12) (status 1000000))
 (segment (start 21.684999 12.794999) (end 17.685001 12.794999) (width 0.25) (layer F.Cu) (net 12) (status 1000000))
 (via (at 31.75 14.605) (size 0.8) (drill 0.4) (layers F.Cu B.Cu) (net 9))
 (segment (start 21.684999 20.225001) (end 19.717001 20.225001) (width 0.25) (layer F.Cu) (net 9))
 (segment (start 22.86 19.05) (end 21.684999 20.225001) (width 0.25) (layer F.Cu) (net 9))
 (segment (start 18.542 19.05) (end 16.51 19.05) (width 0.25) (layer F.Cu) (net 9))
 (segment (start 19.717001 20.225001) (end 18.542 19.05) (width 0.25) (layer F.Cu) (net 9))
 (segment (start 23.81 25.08) (end 22.86 24.13) (width 0.25) (layer F.Cu) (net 9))
 (segment (start 25.67 25.08) (end 23.81 25.08) (width 0.25) (layer F.Cu) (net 9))
 (segment (start 29.226 25.08) (end 25.67 25.08) (width 0.25) (layer F.Cu) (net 9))
 (segment (start 22.86 21.400002) (end 21.684999 20.225001) (width 0.25) (layer F.Cu) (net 9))
 (segment (start 22.86 24.13) (end 22.86 21.400002) (width 0.25) (layer F.Cu) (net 9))
 (segment (start 22.86 19.05) (end 22.86 16.51) (width 0.25) (layer F.Cu) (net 9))
 (segment (start 24.765 14.605) (end 22.86 16.51) (width 0.25) (layer B.Cu) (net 9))
 (segment (start 31.75 14.605) (end 24.765 14.605) (width 0.25) (layer B.Cu) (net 9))
 (segment (start 31.71 14.645) (end 31.75 14.605) (width 0.25) (layer F.Cu) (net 9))
 (segment (start 30.233 14.645) (end 31.71 14.645) (width 0.25) (layer F.Cu) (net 9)))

